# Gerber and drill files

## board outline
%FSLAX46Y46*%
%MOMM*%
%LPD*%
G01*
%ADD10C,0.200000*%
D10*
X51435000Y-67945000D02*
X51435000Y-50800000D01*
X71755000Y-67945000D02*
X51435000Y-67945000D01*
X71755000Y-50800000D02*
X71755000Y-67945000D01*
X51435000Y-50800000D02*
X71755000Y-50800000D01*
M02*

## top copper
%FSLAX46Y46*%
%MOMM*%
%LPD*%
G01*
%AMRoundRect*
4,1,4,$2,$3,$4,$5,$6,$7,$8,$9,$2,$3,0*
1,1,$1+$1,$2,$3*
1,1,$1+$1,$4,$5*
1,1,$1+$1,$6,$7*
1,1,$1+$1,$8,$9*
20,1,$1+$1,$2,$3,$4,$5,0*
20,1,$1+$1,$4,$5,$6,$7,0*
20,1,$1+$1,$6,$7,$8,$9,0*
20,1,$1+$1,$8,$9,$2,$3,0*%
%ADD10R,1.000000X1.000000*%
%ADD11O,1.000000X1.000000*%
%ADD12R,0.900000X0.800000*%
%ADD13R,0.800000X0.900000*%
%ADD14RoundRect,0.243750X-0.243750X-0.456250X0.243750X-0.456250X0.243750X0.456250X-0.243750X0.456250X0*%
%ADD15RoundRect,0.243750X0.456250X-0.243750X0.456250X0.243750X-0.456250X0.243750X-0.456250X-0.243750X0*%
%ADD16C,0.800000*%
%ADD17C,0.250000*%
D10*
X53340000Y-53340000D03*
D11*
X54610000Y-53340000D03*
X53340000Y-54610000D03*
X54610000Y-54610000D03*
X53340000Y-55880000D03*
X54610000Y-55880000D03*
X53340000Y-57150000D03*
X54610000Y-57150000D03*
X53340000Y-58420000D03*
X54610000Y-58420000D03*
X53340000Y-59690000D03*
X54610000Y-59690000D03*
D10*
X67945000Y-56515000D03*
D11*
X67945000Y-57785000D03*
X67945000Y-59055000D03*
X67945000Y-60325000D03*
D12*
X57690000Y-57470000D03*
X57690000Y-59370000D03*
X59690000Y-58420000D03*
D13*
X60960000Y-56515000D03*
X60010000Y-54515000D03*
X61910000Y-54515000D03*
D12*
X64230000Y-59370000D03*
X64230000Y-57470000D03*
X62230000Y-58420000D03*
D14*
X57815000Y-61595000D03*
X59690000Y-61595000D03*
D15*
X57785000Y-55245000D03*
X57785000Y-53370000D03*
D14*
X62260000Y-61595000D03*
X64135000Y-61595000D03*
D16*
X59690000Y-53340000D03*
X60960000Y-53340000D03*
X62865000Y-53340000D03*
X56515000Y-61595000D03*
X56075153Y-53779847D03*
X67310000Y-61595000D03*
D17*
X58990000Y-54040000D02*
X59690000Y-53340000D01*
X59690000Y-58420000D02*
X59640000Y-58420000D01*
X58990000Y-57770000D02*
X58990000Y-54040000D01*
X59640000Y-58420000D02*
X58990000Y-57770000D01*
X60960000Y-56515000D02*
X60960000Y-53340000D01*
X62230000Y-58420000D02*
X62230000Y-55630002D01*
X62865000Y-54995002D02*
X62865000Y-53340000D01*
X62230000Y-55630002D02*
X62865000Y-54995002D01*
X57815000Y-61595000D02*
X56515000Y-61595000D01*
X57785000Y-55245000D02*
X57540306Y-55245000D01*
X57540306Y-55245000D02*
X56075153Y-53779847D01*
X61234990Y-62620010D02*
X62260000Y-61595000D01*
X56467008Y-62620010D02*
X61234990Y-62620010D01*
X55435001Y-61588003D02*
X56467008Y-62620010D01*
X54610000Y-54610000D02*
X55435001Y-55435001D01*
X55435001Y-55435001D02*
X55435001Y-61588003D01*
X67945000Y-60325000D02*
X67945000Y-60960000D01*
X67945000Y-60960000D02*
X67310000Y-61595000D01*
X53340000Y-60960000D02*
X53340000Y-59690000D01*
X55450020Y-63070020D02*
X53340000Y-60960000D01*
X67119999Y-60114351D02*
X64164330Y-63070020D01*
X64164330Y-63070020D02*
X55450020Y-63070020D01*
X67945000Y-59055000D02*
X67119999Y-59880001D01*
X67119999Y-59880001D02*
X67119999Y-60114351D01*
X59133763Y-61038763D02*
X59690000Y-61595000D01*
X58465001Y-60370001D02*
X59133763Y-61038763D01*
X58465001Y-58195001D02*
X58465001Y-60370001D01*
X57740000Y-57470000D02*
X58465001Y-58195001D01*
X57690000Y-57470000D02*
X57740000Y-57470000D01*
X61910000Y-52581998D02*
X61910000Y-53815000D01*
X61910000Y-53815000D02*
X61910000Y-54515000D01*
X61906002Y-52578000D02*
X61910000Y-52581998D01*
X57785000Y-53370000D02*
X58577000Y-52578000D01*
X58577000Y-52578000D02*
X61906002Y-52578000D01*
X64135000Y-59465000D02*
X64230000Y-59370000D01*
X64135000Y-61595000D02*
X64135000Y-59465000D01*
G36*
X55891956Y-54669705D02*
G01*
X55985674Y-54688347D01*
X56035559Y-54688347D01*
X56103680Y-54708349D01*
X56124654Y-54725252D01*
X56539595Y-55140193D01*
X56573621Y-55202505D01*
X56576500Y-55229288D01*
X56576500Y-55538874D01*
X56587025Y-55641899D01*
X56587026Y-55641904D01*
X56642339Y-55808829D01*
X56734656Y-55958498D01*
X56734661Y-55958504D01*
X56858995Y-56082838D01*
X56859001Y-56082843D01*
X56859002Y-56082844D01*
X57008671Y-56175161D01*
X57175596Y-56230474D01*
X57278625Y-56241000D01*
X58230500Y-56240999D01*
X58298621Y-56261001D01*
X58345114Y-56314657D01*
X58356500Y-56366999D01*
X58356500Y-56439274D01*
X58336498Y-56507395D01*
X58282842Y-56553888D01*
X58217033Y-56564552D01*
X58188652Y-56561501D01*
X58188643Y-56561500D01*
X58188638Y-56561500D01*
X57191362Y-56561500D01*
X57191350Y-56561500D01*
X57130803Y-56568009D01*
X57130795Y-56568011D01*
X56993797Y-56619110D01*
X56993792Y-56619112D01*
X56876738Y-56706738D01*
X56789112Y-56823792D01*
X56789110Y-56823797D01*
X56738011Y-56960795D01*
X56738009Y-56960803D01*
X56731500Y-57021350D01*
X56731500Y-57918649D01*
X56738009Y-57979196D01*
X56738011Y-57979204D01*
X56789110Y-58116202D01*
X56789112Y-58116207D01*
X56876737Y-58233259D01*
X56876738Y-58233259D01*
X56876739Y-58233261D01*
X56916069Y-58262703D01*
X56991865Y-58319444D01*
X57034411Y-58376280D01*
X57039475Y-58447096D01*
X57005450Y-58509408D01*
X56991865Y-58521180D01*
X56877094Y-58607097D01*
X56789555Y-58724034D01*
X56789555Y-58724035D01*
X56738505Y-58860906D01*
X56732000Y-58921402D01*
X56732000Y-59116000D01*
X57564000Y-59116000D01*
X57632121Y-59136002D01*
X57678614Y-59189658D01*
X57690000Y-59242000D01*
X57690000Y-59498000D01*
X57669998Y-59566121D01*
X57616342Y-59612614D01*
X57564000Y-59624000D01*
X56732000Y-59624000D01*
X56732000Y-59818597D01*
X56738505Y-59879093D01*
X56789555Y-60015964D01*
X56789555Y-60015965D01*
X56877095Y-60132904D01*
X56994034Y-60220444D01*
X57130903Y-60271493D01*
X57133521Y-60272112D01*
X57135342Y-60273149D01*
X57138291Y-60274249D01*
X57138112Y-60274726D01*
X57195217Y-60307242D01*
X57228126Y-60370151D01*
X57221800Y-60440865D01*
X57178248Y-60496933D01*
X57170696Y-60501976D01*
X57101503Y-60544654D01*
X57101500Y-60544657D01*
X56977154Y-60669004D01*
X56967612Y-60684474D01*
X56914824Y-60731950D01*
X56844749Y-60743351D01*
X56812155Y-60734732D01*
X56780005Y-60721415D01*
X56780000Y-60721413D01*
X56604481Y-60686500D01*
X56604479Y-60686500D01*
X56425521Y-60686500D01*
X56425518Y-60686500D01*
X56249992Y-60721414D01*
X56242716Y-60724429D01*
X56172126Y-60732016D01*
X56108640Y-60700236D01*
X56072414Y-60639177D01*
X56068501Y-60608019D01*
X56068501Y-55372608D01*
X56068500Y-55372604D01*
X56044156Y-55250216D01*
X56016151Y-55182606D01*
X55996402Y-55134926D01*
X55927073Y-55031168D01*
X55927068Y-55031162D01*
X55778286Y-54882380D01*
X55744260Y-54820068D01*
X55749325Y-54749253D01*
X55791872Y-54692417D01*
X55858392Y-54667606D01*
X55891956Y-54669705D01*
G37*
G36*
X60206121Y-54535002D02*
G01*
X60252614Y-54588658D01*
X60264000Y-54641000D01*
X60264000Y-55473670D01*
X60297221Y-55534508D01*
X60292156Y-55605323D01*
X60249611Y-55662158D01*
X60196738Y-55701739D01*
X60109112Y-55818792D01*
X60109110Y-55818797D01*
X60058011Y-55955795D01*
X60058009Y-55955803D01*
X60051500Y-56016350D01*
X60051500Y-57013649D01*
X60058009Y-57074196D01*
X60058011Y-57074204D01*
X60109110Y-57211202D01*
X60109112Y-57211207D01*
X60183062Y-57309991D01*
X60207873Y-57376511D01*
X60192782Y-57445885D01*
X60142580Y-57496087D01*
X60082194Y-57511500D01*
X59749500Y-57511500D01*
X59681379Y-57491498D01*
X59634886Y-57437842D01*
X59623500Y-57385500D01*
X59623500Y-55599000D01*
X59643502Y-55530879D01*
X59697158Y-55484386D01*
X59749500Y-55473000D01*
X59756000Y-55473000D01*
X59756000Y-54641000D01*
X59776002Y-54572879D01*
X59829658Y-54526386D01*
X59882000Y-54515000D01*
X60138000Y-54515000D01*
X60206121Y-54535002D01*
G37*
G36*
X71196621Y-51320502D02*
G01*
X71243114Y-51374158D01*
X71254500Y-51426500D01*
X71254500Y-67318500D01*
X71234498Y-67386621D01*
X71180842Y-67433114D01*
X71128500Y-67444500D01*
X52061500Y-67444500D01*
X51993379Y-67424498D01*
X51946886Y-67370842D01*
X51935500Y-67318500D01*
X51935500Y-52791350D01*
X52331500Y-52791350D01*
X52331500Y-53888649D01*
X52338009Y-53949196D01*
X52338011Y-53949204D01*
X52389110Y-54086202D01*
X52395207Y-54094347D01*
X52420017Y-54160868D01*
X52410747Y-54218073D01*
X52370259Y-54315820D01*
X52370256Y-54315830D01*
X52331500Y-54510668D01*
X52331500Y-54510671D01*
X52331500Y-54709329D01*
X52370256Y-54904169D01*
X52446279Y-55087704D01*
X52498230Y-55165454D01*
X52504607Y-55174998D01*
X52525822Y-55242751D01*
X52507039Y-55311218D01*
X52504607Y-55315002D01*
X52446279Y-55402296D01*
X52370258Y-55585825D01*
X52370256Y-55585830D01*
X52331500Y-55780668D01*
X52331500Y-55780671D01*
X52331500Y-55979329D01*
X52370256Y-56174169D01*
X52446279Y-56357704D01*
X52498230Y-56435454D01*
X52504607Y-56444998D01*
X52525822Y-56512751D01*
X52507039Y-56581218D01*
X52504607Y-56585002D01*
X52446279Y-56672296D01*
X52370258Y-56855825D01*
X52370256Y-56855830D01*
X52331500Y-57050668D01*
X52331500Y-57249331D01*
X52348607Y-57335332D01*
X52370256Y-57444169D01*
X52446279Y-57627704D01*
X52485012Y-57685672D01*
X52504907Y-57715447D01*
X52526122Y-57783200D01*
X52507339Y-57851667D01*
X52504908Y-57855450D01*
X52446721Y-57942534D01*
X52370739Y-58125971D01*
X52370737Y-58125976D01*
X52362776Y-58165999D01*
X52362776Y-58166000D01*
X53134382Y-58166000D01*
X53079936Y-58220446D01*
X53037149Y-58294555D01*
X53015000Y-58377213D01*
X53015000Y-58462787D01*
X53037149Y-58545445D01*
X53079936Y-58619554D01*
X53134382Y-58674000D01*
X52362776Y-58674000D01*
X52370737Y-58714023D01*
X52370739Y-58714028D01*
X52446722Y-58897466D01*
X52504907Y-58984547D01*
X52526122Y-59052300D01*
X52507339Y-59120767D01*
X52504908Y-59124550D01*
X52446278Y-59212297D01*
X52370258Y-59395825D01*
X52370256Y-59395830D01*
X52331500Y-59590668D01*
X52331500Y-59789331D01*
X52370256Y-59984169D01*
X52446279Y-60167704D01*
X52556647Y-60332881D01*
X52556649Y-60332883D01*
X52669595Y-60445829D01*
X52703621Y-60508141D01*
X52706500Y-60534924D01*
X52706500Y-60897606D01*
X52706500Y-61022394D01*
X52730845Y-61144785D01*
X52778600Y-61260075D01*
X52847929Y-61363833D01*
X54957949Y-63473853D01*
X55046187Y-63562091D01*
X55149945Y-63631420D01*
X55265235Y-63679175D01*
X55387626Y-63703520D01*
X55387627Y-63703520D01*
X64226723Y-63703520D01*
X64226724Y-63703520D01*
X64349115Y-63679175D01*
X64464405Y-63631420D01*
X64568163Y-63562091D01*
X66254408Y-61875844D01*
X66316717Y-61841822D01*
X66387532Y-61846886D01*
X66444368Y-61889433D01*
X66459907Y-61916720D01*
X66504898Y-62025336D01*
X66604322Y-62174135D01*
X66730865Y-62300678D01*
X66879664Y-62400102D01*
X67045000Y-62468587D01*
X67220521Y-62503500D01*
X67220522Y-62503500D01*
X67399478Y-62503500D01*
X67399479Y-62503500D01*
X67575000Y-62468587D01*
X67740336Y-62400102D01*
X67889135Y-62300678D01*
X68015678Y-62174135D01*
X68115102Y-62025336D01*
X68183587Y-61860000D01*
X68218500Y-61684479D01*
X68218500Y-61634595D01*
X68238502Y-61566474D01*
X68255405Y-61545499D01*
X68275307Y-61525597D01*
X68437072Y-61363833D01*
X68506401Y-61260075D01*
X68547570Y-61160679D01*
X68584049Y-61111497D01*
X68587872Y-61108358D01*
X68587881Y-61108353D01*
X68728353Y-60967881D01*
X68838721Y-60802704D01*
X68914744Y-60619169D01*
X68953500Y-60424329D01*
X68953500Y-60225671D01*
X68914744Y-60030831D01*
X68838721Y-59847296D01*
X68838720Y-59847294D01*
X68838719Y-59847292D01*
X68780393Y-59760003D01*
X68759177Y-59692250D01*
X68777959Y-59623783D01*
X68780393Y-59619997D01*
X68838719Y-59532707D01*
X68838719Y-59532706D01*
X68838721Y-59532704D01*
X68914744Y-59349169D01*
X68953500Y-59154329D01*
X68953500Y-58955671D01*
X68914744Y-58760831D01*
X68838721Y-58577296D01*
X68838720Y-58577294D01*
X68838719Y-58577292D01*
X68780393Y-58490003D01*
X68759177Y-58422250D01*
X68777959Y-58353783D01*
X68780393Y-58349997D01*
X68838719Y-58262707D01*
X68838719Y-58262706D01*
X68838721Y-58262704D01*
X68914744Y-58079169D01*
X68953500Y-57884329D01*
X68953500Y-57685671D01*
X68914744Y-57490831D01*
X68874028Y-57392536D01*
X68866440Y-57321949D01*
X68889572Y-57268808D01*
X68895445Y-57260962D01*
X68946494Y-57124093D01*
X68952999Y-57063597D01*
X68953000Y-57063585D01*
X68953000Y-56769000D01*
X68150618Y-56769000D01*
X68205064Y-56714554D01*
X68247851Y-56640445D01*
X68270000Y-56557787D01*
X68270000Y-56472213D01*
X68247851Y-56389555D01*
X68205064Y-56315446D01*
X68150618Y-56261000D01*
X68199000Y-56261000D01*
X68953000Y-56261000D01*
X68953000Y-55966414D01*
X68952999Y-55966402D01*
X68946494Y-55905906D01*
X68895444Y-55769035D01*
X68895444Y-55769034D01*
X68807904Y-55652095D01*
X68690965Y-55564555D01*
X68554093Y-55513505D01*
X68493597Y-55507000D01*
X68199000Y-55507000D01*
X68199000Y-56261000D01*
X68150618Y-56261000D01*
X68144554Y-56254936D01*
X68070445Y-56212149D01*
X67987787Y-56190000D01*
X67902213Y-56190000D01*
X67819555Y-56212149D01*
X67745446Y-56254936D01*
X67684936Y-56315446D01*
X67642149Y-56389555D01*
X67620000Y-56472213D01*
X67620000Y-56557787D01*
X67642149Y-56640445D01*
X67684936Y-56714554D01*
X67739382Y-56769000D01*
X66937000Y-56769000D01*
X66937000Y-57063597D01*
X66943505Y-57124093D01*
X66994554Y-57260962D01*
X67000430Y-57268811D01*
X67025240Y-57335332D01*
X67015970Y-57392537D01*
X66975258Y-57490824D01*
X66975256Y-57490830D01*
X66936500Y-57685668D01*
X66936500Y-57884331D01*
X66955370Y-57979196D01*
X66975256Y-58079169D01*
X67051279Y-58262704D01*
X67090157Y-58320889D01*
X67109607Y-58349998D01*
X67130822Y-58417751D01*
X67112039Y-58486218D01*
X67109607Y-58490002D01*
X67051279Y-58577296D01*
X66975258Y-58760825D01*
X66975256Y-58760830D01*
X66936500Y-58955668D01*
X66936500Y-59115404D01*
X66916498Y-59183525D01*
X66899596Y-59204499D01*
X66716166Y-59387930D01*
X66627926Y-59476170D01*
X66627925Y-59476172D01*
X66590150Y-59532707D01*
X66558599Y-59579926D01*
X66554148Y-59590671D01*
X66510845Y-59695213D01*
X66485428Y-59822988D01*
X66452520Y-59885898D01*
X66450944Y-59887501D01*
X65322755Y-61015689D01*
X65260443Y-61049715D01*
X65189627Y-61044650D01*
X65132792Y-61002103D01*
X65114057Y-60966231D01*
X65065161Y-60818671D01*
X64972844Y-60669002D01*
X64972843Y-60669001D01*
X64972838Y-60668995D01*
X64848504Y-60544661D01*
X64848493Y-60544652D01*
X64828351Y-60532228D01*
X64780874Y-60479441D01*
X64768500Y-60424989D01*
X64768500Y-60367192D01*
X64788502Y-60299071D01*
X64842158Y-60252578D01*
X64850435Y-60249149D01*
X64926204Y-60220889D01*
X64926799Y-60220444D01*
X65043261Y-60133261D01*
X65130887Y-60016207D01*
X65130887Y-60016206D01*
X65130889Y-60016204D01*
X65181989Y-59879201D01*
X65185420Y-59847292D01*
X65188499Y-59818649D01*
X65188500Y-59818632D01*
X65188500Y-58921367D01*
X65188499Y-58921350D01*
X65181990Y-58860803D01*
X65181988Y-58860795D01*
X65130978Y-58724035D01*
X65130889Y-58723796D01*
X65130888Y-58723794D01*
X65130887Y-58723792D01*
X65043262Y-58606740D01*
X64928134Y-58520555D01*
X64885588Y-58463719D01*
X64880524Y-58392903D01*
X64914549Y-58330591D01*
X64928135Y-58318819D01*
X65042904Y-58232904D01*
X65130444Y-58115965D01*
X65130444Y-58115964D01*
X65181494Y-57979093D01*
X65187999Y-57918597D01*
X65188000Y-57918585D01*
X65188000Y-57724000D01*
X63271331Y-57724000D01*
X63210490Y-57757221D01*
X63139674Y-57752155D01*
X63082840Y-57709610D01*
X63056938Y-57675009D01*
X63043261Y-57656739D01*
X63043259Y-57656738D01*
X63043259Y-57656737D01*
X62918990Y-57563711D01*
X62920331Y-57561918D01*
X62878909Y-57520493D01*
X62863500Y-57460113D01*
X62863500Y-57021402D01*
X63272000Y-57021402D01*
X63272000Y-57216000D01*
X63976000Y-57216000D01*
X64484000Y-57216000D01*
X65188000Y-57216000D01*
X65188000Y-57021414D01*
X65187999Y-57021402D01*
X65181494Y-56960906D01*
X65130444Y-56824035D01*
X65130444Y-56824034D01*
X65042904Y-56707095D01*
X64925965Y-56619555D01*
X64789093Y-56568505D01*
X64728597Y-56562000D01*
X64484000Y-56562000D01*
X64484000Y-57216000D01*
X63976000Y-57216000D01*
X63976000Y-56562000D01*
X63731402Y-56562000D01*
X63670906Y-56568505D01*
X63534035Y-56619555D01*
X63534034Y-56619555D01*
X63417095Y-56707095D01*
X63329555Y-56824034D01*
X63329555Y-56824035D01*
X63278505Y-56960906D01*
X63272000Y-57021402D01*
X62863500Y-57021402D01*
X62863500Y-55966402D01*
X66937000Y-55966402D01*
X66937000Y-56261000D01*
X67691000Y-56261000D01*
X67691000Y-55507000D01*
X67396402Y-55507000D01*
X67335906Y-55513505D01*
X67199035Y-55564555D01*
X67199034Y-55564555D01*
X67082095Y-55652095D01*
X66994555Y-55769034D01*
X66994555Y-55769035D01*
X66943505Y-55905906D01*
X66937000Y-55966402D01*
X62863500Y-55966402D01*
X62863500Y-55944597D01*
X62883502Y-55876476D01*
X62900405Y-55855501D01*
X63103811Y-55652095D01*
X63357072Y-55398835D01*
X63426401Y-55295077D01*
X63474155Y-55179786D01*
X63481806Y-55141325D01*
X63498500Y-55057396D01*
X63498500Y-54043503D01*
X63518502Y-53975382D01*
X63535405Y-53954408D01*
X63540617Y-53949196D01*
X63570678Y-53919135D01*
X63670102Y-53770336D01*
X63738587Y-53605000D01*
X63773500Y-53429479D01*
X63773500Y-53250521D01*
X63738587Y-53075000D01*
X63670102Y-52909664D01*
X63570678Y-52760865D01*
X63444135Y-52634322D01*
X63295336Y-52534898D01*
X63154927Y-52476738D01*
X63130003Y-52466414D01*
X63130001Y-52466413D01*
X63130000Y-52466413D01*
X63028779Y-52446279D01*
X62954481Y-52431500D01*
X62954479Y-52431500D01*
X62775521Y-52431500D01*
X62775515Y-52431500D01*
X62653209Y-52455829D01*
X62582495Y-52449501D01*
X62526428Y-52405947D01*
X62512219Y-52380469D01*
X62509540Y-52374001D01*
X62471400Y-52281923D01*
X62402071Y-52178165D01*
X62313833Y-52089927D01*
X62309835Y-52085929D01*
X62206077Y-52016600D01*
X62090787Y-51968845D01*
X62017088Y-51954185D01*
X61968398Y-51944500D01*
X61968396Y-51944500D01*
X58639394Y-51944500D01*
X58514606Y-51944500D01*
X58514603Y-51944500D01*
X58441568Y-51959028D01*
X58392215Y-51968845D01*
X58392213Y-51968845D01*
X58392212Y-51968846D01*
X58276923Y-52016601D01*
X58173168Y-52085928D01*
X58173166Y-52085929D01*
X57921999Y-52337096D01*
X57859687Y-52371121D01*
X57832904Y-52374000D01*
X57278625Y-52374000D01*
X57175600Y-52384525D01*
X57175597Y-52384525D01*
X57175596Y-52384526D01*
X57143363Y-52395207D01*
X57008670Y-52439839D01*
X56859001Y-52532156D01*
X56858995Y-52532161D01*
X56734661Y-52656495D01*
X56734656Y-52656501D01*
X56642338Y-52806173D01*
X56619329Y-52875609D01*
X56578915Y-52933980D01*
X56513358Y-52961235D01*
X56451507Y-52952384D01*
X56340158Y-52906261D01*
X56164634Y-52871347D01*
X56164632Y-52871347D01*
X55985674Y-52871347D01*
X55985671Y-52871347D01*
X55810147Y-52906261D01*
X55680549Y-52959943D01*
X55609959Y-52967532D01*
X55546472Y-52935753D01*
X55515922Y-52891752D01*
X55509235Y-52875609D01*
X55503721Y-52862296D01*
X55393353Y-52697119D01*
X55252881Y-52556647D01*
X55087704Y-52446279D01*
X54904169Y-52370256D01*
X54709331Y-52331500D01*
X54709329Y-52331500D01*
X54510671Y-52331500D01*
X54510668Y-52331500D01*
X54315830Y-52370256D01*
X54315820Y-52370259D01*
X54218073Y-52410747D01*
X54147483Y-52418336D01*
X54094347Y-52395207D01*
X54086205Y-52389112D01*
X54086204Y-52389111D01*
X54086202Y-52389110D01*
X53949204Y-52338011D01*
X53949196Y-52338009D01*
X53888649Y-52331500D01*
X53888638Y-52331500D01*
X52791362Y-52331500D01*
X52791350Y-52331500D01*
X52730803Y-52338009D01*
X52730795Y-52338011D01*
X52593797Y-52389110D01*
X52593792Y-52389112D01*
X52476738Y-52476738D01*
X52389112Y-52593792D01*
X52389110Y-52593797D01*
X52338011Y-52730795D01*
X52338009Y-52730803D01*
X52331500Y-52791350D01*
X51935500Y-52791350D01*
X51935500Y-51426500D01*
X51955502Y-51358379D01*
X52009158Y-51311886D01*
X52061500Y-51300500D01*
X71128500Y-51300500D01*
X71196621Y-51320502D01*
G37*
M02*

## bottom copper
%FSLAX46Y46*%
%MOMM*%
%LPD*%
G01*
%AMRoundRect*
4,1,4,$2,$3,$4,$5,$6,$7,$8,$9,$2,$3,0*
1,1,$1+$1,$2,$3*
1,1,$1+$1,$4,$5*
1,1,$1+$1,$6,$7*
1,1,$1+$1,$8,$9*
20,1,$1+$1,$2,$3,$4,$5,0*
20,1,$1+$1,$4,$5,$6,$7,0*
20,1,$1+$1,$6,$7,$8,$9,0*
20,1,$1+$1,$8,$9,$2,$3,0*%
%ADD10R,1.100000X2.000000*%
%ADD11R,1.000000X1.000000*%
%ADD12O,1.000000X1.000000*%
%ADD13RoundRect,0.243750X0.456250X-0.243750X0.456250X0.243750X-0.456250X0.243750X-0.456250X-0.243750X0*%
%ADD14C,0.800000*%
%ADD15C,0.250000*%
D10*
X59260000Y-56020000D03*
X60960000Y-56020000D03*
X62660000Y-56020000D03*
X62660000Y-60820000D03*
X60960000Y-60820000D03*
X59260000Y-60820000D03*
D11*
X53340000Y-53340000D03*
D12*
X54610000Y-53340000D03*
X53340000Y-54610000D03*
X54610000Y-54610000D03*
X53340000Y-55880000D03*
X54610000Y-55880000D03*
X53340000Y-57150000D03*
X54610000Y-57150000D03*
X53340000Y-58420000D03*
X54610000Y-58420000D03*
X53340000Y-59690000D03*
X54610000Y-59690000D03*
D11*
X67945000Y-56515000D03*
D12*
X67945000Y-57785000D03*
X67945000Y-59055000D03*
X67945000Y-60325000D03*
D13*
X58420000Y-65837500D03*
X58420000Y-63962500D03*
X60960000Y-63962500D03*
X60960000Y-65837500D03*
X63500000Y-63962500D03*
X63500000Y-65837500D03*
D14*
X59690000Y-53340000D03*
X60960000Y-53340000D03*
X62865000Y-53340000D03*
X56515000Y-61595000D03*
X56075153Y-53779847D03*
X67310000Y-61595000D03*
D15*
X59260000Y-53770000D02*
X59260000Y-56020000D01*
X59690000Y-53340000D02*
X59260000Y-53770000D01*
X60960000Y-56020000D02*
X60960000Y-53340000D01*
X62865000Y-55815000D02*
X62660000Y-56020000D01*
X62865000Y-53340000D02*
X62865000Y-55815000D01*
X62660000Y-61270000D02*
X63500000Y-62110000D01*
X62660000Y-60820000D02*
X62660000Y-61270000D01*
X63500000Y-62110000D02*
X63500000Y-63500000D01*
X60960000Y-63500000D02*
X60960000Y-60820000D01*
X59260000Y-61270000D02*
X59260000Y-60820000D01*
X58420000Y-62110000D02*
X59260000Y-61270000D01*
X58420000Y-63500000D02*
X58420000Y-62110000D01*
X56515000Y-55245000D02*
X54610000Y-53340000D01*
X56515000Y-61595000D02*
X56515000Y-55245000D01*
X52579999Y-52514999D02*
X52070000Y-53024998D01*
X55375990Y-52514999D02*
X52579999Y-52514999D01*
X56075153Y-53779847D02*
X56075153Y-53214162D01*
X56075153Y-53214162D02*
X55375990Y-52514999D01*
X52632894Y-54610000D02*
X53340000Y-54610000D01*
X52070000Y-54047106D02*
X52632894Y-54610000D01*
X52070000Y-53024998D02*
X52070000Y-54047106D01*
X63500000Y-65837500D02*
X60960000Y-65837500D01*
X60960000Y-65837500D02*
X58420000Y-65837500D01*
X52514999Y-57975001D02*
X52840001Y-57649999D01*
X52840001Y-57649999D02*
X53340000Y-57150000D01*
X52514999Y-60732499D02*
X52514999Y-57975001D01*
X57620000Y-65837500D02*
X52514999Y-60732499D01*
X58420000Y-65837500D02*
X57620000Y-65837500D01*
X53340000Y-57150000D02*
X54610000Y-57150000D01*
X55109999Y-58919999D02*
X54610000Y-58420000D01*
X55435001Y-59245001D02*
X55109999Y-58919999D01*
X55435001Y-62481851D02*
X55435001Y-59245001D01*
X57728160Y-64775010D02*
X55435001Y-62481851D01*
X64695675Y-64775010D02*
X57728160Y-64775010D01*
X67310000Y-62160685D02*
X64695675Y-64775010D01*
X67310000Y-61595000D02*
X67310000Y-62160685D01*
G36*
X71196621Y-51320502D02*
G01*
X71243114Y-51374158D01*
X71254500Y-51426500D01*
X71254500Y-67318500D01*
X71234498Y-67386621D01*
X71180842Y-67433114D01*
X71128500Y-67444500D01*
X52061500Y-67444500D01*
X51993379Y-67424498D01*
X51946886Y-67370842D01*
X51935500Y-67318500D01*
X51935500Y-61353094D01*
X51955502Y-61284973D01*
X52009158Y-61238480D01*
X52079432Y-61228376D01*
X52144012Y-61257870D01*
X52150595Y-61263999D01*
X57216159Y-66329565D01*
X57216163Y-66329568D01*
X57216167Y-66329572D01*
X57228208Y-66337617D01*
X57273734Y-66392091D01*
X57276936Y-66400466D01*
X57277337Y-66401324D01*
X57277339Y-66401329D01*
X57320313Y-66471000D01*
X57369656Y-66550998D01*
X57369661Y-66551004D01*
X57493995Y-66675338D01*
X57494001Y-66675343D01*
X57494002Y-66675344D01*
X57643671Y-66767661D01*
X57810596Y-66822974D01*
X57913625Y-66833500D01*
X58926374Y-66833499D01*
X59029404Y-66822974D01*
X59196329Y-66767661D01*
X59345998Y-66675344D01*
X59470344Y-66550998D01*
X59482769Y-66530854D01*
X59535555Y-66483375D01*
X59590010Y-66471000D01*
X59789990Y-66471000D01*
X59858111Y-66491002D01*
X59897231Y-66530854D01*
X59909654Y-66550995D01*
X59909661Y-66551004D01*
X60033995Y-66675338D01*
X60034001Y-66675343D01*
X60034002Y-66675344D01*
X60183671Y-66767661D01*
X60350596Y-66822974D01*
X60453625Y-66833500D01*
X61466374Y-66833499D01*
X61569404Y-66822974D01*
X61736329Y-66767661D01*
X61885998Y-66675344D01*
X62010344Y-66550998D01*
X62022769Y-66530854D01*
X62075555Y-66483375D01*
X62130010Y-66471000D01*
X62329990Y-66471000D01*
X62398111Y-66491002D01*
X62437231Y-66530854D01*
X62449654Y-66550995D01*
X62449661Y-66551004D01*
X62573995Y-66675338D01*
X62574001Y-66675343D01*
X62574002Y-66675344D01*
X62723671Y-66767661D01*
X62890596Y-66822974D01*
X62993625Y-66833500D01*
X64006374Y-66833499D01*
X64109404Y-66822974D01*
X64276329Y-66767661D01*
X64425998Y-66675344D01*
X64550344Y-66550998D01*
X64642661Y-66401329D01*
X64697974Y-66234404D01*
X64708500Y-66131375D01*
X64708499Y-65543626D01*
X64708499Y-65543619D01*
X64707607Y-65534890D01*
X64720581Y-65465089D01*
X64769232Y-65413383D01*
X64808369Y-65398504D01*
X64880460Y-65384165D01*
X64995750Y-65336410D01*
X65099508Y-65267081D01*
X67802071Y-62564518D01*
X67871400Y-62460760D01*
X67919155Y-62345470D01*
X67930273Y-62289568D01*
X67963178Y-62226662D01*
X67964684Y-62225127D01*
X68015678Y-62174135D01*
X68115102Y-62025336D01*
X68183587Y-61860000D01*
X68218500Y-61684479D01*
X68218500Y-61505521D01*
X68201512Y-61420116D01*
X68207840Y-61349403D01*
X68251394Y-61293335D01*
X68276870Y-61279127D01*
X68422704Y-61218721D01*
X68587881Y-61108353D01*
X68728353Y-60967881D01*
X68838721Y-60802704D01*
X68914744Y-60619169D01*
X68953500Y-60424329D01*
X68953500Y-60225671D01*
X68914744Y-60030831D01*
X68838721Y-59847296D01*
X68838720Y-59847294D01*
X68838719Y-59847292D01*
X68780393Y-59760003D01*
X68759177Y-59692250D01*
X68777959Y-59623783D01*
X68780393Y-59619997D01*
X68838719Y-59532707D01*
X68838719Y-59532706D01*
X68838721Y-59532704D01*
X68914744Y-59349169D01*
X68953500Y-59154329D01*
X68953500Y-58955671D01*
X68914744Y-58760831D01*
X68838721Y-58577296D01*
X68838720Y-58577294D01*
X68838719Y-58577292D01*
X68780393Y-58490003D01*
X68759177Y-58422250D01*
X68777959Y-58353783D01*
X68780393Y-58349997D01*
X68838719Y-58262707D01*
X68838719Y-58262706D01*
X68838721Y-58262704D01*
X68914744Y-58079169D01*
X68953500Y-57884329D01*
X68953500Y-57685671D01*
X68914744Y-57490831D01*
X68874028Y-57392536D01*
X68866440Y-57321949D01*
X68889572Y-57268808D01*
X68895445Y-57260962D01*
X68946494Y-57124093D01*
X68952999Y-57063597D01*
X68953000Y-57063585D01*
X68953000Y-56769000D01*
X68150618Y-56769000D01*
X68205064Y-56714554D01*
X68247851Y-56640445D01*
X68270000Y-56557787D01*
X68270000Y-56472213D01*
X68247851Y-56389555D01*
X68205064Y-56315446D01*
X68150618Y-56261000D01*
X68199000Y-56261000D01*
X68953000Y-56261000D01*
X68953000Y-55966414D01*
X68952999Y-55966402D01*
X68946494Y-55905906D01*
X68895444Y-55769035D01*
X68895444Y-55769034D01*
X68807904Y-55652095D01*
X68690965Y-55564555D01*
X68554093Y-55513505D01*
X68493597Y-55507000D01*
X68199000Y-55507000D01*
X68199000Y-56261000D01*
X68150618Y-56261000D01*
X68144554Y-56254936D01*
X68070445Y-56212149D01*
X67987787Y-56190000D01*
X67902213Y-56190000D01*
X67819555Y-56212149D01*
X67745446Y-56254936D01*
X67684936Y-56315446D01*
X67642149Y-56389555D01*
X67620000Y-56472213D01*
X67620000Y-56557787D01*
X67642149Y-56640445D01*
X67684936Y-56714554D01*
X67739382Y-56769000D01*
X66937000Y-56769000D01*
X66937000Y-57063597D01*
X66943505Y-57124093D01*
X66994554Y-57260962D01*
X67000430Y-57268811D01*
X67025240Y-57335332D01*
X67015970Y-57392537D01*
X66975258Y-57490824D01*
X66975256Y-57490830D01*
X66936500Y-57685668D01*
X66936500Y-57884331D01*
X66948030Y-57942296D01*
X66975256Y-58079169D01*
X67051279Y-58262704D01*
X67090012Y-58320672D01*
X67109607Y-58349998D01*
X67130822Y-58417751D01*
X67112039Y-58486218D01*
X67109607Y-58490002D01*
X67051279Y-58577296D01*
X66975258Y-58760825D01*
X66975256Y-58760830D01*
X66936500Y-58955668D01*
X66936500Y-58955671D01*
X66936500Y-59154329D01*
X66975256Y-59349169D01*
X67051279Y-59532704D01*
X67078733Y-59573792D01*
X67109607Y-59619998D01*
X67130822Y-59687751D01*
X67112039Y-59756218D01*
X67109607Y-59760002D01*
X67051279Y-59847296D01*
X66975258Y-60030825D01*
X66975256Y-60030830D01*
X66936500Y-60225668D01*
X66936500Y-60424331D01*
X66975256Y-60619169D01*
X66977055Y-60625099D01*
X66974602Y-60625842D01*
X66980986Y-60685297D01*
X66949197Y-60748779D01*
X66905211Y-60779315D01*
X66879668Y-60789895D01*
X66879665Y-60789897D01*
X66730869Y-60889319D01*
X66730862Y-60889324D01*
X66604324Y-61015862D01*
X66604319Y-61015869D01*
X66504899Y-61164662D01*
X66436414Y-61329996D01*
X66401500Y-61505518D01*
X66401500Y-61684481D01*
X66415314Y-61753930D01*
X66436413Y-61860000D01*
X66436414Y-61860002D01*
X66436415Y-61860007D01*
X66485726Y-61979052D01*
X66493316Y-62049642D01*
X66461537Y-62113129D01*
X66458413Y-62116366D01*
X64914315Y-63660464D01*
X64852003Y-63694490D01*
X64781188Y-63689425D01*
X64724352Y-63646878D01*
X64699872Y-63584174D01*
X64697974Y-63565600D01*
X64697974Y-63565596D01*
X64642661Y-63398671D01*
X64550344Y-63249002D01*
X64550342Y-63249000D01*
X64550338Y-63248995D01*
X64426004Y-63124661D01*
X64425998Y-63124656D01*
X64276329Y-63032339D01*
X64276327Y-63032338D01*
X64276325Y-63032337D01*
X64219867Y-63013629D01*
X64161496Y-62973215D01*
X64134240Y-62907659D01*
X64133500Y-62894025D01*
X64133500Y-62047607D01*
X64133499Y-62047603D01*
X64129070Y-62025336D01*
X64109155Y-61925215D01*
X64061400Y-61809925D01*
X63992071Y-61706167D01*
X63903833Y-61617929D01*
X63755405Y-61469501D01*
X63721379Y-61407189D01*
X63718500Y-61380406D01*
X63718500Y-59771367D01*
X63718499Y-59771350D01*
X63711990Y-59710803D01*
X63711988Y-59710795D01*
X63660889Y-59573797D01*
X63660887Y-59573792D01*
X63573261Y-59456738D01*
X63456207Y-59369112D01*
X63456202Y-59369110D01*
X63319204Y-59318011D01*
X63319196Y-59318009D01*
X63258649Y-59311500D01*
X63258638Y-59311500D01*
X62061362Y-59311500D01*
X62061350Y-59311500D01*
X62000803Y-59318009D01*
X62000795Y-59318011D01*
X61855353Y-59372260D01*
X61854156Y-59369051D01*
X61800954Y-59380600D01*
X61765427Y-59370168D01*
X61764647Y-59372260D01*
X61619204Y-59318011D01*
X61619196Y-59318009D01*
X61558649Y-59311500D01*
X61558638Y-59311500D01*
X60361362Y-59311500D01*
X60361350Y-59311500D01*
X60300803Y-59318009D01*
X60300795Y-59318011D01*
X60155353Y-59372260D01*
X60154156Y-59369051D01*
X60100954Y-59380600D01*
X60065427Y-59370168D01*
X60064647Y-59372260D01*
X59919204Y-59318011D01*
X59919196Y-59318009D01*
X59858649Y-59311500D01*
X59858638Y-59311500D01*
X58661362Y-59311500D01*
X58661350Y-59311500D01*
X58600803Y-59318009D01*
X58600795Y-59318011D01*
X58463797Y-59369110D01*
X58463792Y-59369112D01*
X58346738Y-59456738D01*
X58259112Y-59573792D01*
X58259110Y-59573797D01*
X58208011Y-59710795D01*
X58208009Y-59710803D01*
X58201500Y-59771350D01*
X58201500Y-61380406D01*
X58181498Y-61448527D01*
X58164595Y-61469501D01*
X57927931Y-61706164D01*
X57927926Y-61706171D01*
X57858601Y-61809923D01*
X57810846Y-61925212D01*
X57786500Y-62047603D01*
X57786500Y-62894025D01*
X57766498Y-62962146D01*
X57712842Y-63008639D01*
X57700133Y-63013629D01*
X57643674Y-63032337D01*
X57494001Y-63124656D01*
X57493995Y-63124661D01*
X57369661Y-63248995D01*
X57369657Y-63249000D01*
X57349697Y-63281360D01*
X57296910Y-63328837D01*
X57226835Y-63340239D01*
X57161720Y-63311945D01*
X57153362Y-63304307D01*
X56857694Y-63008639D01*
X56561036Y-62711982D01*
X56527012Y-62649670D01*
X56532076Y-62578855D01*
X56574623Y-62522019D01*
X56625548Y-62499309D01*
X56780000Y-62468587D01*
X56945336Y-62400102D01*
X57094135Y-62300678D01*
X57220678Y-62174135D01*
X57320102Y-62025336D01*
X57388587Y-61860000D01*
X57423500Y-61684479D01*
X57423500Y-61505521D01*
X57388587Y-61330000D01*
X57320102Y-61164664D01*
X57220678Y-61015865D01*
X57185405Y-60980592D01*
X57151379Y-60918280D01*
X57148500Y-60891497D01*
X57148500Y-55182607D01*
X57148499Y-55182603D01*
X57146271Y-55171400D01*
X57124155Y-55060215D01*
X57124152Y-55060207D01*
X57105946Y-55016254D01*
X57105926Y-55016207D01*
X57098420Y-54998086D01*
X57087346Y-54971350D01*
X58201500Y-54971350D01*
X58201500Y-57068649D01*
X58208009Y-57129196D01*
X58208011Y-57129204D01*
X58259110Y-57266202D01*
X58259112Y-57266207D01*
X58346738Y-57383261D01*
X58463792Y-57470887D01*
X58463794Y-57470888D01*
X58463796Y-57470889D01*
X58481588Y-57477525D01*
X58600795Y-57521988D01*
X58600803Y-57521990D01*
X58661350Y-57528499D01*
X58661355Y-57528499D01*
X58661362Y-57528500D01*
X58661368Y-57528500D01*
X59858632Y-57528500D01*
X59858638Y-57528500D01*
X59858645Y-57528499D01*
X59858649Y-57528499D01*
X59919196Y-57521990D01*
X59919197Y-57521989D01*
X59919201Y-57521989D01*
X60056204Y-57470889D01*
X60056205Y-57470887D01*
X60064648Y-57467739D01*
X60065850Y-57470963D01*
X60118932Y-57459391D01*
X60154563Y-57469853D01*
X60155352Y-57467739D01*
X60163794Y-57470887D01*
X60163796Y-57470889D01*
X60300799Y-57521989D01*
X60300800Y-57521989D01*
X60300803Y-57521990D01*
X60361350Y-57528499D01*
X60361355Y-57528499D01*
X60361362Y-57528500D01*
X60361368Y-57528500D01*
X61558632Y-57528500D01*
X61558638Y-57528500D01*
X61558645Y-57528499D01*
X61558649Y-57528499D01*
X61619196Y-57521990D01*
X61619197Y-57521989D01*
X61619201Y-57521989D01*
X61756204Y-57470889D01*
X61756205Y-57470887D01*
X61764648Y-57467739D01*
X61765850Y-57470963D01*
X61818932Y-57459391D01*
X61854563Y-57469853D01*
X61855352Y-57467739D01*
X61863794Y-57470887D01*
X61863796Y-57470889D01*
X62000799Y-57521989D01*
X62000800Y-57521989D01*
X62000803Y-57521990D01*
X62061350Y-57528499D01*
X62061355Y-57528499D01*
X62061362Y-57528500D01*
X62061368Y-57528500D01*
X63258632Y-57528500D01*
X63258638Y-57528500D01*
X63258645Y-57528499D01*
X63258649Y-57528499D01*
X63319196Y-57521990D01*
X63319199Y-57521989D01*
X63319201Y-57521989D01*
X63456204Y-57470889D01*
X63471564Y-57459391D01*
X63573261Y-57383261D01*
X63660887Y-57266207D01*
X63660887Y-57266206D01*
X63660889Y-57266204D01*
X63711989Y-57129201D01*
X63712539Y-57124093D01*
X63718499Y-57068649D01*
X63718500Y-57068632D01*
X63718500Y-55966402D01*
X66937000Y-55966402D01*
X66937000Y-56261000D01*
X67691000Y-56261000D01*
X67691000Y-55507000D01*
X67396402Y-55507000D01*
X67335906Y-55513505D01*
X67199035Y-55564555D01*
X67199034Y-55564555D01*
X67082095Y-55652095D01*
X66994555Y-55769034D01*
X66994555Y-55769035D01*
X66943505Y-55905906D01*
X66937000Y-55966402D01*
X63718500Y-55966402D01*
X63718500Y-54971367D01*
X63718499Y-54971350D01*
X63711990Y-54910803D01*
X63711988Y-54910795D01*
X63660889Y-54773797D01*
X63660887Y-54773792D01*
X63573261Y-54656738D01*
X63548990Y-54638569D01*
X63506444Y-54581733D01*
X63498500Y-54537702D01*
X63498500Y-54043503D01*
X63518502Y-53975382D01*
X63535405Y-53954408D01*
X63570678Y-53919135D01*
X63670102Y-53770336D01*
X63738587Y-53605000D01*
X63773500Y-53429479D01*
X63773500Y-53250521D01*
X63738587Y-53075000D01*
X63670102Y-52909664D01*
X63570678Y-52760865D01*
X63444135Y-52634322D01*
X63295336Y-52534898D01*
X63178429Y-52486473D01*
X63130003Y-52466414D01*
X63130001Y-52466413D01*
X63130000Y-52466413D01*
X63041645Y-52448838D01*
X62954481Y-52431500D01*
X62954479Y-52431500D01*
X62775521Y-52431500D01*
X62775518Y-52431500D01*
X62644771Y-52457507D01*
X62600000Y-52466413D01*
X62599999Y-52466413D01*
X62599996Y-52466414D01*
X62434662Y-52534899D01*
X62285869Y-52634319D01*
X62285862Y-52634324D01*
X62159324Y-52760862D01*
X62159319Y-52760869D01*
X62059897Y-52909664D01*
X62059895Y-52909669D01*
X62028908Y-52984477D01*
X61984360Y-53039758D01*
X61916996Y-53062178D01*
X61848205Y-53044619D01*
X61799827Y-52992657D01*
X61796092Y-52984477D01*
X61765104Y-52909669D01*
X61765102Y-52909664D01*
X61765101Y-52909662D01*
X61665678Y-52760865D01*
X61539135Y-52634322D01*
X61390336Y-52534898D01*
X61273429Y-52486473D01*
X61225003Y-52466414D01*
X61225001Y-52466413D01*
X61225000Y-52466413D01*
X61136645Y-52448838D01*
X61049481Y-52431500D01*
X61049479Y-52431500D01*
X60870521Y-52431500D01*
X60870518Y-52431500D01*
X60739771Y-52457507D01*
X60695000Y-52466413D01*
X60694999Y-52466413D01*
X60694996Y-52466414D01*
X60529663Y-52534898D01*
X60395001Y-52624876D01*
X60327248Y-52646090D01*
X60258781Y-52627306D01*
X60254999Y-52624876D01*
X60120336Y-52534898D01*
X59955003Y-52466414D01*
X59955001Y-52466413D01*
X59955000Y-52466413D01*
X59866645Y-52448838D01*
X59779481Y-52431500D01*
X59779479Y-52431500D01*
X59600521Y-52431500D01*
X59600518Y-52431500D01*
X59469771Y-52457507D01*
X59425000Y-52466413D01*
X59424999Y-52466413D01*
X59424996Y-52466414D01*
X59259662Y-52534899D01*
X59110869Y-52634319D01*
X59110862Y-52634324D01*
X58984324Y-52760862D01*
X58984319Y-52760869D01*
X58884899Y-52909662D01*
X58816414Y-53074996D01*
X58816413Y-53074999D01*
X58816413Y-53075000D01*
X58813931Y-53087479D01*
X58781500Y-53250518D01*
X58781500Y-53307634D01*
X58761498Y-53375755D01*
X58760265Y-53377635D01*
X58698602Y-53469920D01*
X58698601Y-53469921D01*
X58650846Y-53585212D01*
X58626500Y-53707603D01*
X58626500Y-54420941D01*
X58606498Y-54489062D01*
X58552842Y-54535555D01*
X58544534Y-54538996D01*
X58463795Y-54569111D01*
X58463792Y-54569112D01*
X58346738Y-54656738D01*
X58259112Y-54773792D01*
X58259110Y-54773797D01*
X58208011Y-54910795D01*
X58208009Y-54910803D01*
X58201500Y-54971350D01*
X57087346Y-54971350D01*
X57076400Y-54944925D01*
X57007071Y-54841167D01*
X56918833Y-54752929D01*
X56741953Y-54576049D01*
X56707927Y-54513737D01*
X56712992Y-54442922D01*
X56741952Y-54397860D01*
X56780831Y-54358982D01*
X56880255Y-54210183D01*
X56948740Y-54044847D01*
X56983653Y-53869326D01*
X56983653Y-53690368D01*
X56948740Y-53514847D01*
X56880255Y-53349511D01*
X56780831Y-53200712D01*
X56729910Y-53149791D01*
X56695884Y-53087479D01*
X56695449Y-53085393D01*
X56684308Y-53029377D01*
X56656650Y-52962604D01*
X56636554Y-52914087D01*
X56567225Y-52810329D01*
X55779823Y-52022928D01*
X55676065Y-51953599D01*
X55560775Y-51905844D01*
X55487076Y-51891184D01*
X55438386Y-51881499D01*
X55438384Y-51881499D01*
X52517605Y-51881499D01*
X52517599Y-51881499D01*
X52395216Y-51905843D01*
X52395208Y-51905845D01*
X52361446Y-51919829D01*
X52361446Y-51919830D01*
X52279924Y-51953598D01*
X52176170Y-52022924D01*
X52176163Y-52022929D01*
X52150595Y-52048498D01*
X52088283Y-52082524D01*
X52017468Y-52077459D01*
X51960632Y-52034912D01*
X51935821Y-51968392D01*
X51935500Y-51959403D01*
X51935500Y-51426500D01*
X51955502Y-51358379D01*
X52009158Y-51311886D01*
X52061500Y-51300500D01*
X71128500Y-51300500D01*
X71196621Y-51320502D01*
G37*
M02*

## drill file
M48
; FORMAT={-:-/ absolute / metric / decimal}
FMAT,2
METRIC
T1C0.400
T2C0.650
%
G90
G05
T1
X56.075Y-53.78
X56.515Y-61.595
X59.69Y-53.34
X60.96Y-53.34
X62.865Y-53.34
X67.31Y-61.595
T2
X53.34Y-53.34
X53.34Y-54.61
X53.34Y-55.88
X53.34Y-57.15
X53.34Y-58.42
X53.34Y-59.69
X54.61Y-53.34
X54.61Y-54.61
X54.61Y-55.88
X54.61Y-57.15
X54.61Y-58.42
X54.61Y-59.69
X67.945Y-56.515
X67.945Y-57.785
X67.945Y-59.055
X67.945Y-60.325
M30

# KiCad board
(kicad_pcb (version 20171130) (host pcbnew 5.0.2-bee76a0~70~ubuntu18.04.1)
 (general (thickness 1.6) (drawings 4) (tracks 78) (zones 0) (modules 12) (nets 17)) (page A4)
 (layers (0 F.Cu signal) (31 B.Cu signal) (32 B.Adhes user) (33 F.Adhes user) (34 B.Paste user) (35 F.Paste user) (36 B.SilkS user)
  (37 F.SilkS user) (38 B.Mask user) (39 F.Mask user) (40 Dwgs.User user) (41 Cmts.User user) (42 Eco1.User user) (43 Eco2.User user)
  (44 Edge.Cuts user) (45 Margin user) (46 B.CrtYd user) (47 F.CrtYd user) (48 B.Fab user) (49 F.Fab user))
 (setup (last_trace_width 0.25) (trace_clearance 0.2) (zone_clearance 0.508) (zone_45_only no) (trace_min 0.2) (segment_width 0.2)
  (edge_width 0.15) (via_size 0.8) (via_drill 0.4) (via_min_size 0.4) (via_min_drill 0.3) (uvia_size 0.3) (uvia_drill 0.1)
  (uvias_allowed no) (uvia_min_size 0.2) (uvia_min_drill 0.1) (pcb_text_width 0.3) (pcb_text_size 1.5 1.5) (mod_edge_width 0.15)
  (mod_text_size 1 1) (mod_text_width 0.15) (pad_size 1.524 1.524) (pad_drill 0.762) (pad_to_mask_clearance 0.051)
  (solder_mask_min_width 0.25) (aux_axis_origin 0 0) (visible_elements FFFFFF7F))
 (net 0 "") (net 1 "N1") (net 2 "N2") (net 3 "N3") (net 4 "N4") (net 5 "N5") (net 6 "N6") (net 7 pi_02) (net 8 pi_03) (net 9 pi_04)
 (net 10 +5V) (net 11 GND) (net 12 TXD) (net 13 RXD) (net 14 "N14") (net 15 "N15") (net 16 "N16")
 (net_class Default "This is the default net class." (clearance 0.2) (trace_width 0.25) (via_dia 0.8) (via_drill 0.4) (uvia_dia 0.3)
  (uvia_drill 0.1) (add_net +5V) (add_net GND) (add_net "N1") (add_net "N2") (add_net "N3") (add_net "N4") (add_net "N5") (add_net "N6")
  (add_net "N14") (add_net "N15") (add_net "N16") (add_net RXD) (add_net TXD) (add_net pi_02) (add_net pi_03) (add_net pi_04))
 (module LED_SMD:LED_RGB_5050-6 (layer B.Cu) (at 60.96 58.42 270)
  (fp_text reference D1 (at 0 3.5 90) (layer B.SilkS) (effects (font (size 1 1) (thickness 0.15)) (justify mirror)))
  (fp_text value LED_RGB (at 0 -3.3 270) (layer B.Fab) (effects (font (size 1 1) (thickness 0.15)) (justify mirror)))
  (pad 1 smd rect (at -2.4 1.7 180) (size 1.1 2) (layers B.Cu B.Paste B.Mask) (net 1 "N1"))
  (pad 2 smd rect (at -2.4 0 180) (size 1.1 2) (layers B.Cu B.Paste B.Mask) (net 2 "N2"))
  (pad 3 smd rect (at -2.4 -1.7 180) (size 1.1 2) (layers B.Cu B.Paste B.Mask) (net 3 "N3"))
  (pad 4 smd rect (at 2.4 -1.7 180) (size 1.1 2) (layers B.Cu B.Paste B.Mask) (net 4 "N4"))
  (pad 5 smd rect (at 2.4 0 180) (size 1.1 2) (layers B.Cu B.Paste B.Mask) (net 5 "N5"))
  (pad 6 smd rect (at 2.4 1.7 180) (size 1.1 2) (layers B.Cu B.Paste B.Mask) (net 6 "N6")))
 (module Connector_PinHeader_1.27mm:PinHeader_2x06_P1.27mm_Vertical (layer F.Cu) (at 53.34 53.34)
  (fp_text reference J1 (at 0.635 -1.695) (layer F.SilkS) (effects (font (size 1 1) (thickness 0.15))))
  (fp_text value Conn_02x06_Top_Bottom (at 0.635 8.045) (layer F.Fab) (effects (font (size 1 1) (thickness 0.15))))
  (pad 1 thru_hole rect (at 0 0) (size 1 1) (drill 0.65) (layers *.Cu *.Mask))
  (pad 2 thru_hole oval (at 1.27 0) (size 1 1) (drill 0.65) (layers *.Cu *.Mask) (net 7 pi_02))
  (pad 3 thru_hole oval (at 0 1.27) (size 1 1) (drill 0.65) (layers *.Cu *.Mask) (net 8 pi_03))
  (pad 4 thru_hole oval (at 1.27 1.27) (size 1 1) (drill 0.65) (layers *.Cu *.Mask) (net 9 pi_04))
  (pad 5 thru_hole oval (at 0 2.54) (size 1 1) (drill 0.65) (layers *.Cu *.Mask))
  (pad 6 thru_hole oval (at 1.27 2.54) (size 1 1) (drill 0.65) (layers *.Cu *.Mask))
  (pad 7 thru_hole oval (at 0 3.81) (size 1 1) (drill 0.65) (layers *.Cu *.Mask) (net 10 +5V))
  (pad 8 thru_hole oval (at 1.27 3.81) (size 1 1) (drill 0.65) (layers *.Cu *.Mask) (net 10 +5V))
  (pad 9 thru_hole oval (at 0 5.08) (size 1 1) (drill 0.65) (layers *.Cu *.Mask) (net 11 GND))
  (pad 10 thru_hole oval (at 1.27 5.08) (size 1 1) (drill 0.65) (layers *.Cu *.Mask) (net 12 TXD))
  (pad 11 thru_hole oval (at 0 6.35) (size 1 1) (drill 0.65) (layers *.Cu *.Mask) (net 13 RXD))
  (pad 12 thru_hole oval (at 1.27 6.35) (size 1 1) (drill 0.65) (layers *.Cu *.Mask)))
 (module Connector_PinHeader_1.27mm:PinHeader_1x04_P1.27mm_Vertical (layer F.Cu) (at 67.945 56.515)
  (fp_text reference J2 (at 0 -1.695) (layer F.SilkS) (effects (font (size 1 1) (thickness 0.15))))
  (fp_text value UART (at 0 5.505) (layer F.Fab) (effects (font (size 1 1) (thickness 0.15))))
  (pad 1 thru_hole rect (at 0 0) (size 1 1) (drill 0.65) (layers *.Cu *.Mask) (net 11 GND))
  (pad 2 thru_hole oval (at 0 1.27) (size 1 1) (drill 0.65) (layers *.Cu *.Mask))
  (pad 3 thru_hole oval (at 0 2.54) (size 1 1) (drill 0.65) (layers *.Cu *.Mask) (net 13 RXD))
  (pad 4 thru_hole oval (at 0 3.81) (size 1 1) (drill 0.65) (layers *.Cu *.Mask) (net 12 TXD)))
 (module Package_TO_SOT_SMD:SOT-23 (layer F.Cu) (at 58.69 58.42)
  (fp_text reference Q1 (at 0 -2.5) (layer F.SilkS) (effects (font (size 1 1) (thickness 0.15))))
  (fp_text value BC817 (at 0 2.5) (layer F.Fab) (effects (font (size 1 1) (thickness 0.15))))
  (pad 1 smd rect (at -1 -0.95) (size 0.9 0.8) (layers F.Cu F.Paste F.Mask) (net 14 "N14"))
  (pad 2 smd rect (at -1 0.95) (size 0.9 0.8) (layers F.Cu F.Paste F.Mask) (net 11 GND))
  (pad 3 smd rect (at 1 0) (size 0.9 0.8) (layers F.Cu F.Paste F.Mask) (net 1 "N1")))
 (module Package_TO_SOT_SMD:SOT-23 (layer F.Cu) (at 60.96 55.515 270)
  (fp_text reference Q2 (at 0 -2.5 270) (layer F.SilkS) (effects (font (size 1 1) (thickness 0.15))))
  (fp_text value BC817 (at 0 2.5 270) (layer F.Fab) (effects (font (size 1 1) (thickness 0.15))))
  (pad 3 smd rect (at 1 0 270) (size 0.9 0.8) (layers F.Cu F.Paste F.Mask) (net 2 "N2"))
  (pad 2 smd rect (at -1 0.95 270) (size 0.9 0.8) (layers F.Cu F.Paste F.Mask) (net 11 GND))
  (pad 1 smd rect (at -1 -0.95 270) (size 0.9 0.8) (layers F.Cu F.Paste F.Mask) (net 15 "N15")))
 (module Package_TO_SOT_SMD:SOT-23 (layer F.Cu) (at 63.23 58.42 180)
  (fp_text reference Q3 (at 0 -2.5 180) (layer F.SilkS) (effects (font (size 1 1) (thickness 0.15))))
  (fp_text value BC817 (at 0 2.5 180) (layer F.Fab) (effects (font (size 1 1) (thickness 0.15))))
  (pad 1 smd rect (at -1 -0.95 180) (size 0.9 0.8) (layers F.Cu F.Paste F.Mask) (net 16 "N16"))
  (pad 2 smd rect (at -1 0.95 180) (size 0.9 0.8) (layers F.Cu F.Paste F.Mask) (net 11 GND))
  (pad 3 smd rect (at 1 0 180) (size 0.9 0.8) (layers F.Cu F.Paste F.Mask) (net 3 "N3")))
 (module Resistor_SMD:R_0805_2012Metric (layer F.Cu) (at 58.7525 61.595)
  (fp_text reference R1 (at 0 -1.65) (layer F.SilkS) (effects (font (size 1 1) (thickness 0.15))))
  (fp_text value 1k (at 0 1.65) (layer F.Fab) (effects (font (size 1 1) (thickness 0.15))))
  (pad 1 smd roundrect (at -0.9375 0) (size 0.975 1.4) (layers F.Cu F.Paste F.Mask) (roundrect_rratio 0.25) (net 7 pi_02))
  (pad 2 smd roundrect (at 0.9375 0) (size 0.975 1.4) (layers F.Cu F.Paste F.Mask) (roundrect_rratio 0.25) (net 14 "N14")))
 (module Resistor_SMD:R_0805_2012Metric (layer F.Cu) (at 57.785 54.3075 90)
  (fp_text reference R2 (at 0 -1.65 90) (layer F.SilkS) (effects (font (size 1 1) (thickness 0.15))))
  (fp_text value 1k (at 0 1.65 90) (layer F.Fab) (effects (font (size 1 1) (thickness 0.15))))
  (pad 1 smd roundrect (at -0.9375 0 90) (size 0.975 1.4) (layers F.Cu F.Paste F.Mask) (roundrect_rratio 0.25) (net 8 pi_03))
  (pad 2 smd roundrect (at 0.9375 0 90) (size 0.975 1.4) (layers F.Cu F.Paste F.Mask) (roundrect_rratio 0.25) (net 15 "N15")))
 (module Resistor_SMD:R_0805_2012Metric (layer F.Cu) (at 63.1975 61.595)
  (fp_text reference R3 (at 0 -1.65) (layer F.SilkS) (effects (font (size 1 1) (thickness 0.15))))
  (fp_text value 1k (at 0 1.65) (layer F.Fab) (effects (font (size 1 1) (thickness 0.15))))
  (pad 1 smd roundrect (at -0.9375 0) (size 0.975 1.4) (layers F.Cu F.Paste F.Mask) (roundrect_rratio 0.25) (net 9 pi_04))
  (pad 2 smd roundrect (at 0.9375 0) (size 0.975 1.4) (layers F.Cu F.Paste F.Mask) (roundrect_rratio 0.25) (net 16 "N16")))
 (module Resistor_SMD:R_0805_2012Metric (layer B.Cu) (at 58.42 64.9 90)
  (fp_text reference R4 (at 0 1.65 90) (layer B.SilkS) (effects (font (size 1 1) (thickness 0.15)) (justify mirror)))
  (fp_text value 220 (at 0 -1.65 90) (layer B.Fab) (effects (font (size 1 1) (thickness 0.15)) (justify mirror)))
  (pad 1 smd roundrect (at -0.9375 0 90) (size 0.975 1.4) (layers B.Cu B.Paste B.Mask) (roundrect_rratio 0.25) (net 10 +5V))
  (pad 2 smd roundrect (at 0.9375 0 90) (size 0.975 1.4) (layers B.Cu B.Paste B.Mask) (roundrect_rratio 0.25) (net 6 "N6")))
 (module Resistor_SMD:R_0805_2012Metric (layer B.Cu) (at 60.96 64.9 90)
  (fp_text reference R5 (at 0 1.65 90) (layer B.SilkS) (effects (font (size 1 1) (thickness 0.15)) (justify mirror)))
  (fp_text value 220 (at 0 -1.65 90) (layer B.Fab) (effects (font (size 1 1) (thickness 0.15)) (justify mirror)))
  (pad 2 smd roundrect (at 0.9375 0 90) (size 0.975 1.4) (layers B.Cu B.Paste B.Mask) (roundrect_rratio 0.25) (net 5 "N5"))
  (pad 1 smd roundrect (at -0.9375 0 90) (size 0.975 1.4) (layers B.Cu B.Paste B.Mask) (roundrect_rratio 0.25) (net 10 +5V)))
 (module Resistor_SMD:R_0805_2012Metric (layer B.Cu) (at 63.5 64.9 90)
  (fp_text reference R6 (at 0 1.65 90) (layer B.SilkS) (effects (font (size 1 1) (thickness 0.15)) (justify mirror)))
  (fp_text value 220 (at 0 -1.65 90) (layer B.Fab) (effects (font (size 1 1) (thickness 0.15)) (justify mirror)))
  (pad 2 smd roundrect (at 0.9375 0 90) (size 0.975 1.4) (layers B.Cu B.Paste B.Mask) (roundrect_rratio 0.25) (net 4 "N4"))
  (pad 1 smd roundrect (at -0.9375 0 90) (size 0.975 1.4) (layers B.Cu B.Paste B.Mask) (roundrect_rratio 0.25) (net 10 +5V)))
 (gr_line (start 51.435 67.945) (end 51.435 50.8) (layer Edge.Cuts) (width 0.2))
 (gr_line (start 71.755 67.945) (end 51.435 67.945) (layer Edge.Cuts) (width 0.2))
 (gr_line (start 71.755 50.8) (end 71.755 67.945) (layer Edge.Cuts) (width 0.2))
 (gr_line (start 51.435 50.8) (end 71.755 50.8) (layer Edge.Cuts) (width 0.2))
 (segment (start 58.99 54.04) (end 59.69 53.34) (width 0.25) (layer F.Cu) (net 1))
 (segment (start 59.69 58.42) (end 59.64 58.42) (width 0.25) (layer F.Cu) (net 1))
 (via (at 59.69 53.34) (size 0.8) (drill 0.4) (layers F.Cu B.Cu) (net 1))
 (segment (start 58.99 57.77) (end 58.99 54.04) (width 0.25) (layer F.Cu) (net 1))
 (segment (start 59.64 58.42) (end 58.99 57.77) (width 0.25) (layer F.Cu) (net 1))
 (segment (start 59.26 53.77) (end 59.26 56.02) (width 0.25) (layer B.Cu) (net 1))
 (segment (start 59.69 53.34) (end 59.26 53.77) (width 0.25) (layer B.Cu) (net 1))
 (via (at 60.96 53.34) (size 0.8) (drill 0.4) (layers F.Cu B.Cu) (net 2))
 (segment (start 60.96 56.515) (end 60.96 53.34) (width 0.25) (layer F.Cu) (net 2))
 (segment (start 60.96 56.02) (end 60.96 53.34) (width 0.25) (layer B.Cu) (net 2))
 (via (at 62.865 53.34) (size 0.8) (drill 0.4) (layers F.Cu B.Cu) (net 3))
 (segment (start 62.23 58.42) (end 62.23 55.630002) (width 0.25) (layer F.Cu) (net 3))
 (segment (start 62.865 54.995002) (end 62.865 53.34) (width 0.25) (layer F.Cu) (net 3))
 (segment (start 62.23 55.630002) (end 62.865 54.995002) (width 0.25) (layer F.Cu) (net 3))
 (segment (start 62.865 55.815) (end 62.66 56.02) (width 0.25) (layer B.Cu) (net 3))
 (segment (start 62.865 53.34) (end 62.865 55.815) (width 0.25) (layer B.Cu) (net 3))
 (segment (start 62.66 61.27) (end 63.5 62.11) (width 0.25) (layer B.Cu) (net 4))
 (segment (start 62.66 60.82) (end 62.66 61.27) (width 0.25) (layer B.Cu) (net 4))
 (segment (start 63.5 62.11) (end 63.5 63.5) (width 0.25) (layer B.Cu) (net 4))
 (segment (start 60.96 63.5) (end 60.96 60.82) (width 0.25) (layer B.Cu) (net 5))
 (segment (start 59.26 61.27) (end 59.26 60.82) (width 0.25) (layer B.Cu) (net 6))
 (segment (start 58.42 62.11) (end 59.26 61.27) (width 0.25) (layer B.Cu) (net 6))
 (segment (start 58.42 63.5) (end 58.42 62.11) (width 0.25) (layer B.Cu) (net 6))
 (via (at 56.515 61.595) (size 0.8) (drill 0.4) (layers F.Cu B.Cu) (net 7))
 (segment (start 57.815 61.595) (end 56.515 61.595) (width 0.25) (layer F.Cu) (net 7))
 (segment (start 56.515 55.245) (end 54.61 53.34) (width 0.25) (layer B.Cu) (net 7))
 (segment (start 56.515 61.595) (end 56.515 55.245) (width 0.25) (layer B.Cu) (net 7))
 (via (at 56.075153 53.779847) (size 0.8) (drill 0.4) (layers F.Cu B.Cu) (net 8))
 (segment (start 57.785 55.245) (end 57.540306 55.245) (width 0.25) (layer F.Cu) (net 8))
 (segment (start 57.540306 55.245) (end 56.075153 53.779847) (width 0.25) (layer F.Cu) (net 8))
 (segment (start 52.579999 52.514999) (end 52.07 53.024998) (width 0.25) (layer B.Cu) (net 8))
 (segment (start 55.37599 52.514999) (end 52.579999 52.514999) (width 0.25) (layer B.Cu) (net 8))
 (segment (start 56.075153 53.779847) (end 56.075153 53.214162) (width 0.25) (layer B.Cu) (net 8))
 (segment (start 56.075153 53.214162) (end 55.37599 52.514999) (width 0.25) (layer B.Cu) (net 8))
 (segment (start 52.632894 54.61) (end 53.34 54.61) (width 0.25) (layer B.Cu) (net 8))
 (segment (start 52.07 54.047106) (end 52.632894 54.61) (width 0.25) (layer B.Cu) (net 8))
 (segment (start 52.07 53.024998) (end 52.07 54.047106) (width 0.25) (layer B.Cu) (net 8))
 (segment (start 61.23499 62.62001) (end 62.26 61.595) (width 0.25) (layer F.Cu) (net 9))
 (segment (start 56.467008 62.62001) (end 61.23499 62.62001) (width 0.25) (layer F.Cu) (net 9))
 (segment (start 55.435001 61.588003) (end 56.467008 62.62001) (width 0.25) (layer F.Cu) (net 9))
 (segment (start 54.61 54.61) (end 55.435001 55.435001) (width 0.25) (layer F.Cu) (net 9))
 (segment (start 55.435001 55.435001) (end 55.435001 61.588003) (width 0.25) (layer F.Cu) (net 9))
 (segment (start 63.5 65.8375) (end 60.96 65.8375) (width 0.25) (layer B.Cu) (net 10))
 (segment (start 60.96 65.8375) (end 58.42 65.8375) (width 0.25) (layer B.Cu) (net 10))
 (segment (start 52.514999 57.975001) (end 52.840001 57.649999) (width 0.25) (layer B.Cu) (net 10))
 (segment (start 52.840001 57.649999) (end 53.34 57.15) (width 0.25) (layer B.Cu) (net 10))
 (segment (start 52.514999 60.732499) (end 52.514999 57.975001) (width 0.25) (layer B.Cu) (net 10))
 (segment (start 57.62 65.8375) (end 52.514999 60.732499) (width 0.25) (layer B.Cu) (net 10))
 (segment (start 58.42 65.8375) (end 57.62 65.8375) (width 0.25) (layer B.Cu) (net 10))
 (segment (start 53.34 57.15) (end 54.61 57.15) (width 0.25) (layer B.Cu) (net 10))
 (via (at 67.31 61.595) (size 0.8) (drill 0.4) (layers F.Cu B.Cu) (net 12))
 (segment (start 67.945 60.325) (end 67.945 60.96) (width 0.25) (layer F.Cu) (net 12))
 (segment (start 67.945 60.96) (end 67.31 61.595) (width 0.25) (layer F.Cu) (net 12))
 (segment (start 55.109999 58.919999) (end 54.61 58.42) (width 0.25) (layer B.Cu) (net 12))
 (segment (start 55.435001 59.245001) (end 55.109999 58.919999) (width 0.25) (layer B.Cu) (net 12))
 (segment (start 55.435001 62.481851) (end 55.435001 59.245001) (width 0.25) (layer B.Cu) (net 12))
 (segment (start 57.72816 64.77501) (end 55.435001 62.481851) (width 0.25) (layer B.Cu) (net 12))
 (segment (start 64.695675 64.77501) (end 57.72816 64.77501) (width 0.25) (layer B.Cu) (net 12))
 (segment (start 67.31 62.160685) (end 64.695675 64.77501) (width 0.25) (layer B.Cu) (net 12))
 (segment (start 67.31 61.595) (end 67.31 62.160685) (width 0.25) (layer B.Cu) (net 12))
 (segment (start 53.34 60.96) (end 53.34 59.69) (width 0.25) (layer F.Cu) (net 13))
 (segment (start 55.45002 63.07002) (end 53.34 60.96) (width 0.25) (layer F.Cu) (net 13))
 (segment (start 67.119999 60.114351) (end 64.16433 63.07002) (width 0.25) (layer F.Cu) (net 13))
 (segment (start 64.16433 63.07002) (end 55.45002 63.07002) (width 0.25) (layer F.Cu) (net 13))
 (segment (start 67.945 59.055) (end 67.119999 59.880001) (width 0.25) (layer F.Cu) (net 13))
 (segment (start 67.119999 59.880001) (end 67.119999 60.114351) (width 0.25) (layer F.Cu) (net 13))
 (segment (start 59.133763 61.038763) (end 59.69 61.595) (width 0.25) (layer F.Cu) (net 14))
 (segment (start 58.465001 60.370001) (end 59.133763 61.038763) (width 0.25) (layer F.Cu) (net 14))
 (segment (start 58.465001 58.195001) (end 58.465001 60.370001) (width 0.25) (layer F.Cu) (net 14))
 (segment (start 57.74 57.47) (end 58.465001 58.195001) (width 0.25) (layer F.Cu) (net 14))
 (segment (start 57.69 57.47) (end 57.74 57.47) (width 0.25) (layer F.Cu) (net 14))
 (segment (start 61.91 52.581998) (end 61.91 53.815) (width 0.25) (layer F.Cu) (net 15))
 (segment (start 61.91 53.815) (end 61.91 54.515) (width 0.25) (layer F.Cu) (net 15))
 (segment (start 61.906002 52.578) (end 61.91 52.581998) (width 0.25) (layer F.Cu) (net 15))
 (segment (start 57.785 53.37) (end 58.577 52.578) (width 0.25) (layer F.Cu) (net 15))
 (segment (start 58.577 52.578) (end 61.906002 52.578) (width 0.25) (layer F.Cu) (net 15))
 (segment (start 64.135 59.465) (end 64.23 59.37) (width 0.25) (layer F.Cu) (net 16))
 (segment (start 64.135 61.595) (end 64.135 59.465) (width 0.25) (layer F.Cu) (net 16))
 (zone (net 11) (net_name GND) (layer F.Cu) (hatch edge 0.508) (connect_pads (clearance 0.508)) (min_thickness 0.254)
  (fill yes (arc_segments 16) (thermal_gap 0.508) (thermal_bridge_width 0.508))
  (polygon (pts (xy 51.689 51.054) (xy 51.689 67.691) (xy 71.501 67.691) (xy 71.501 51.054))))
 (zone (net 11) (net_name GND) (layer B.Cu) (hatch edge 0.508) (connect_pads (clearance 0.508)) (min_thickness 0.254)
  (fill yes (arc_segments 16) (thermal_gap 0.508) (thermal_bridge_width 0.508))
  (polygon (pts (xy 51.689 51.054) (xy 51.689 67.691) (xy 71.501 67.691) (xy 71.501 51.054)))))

